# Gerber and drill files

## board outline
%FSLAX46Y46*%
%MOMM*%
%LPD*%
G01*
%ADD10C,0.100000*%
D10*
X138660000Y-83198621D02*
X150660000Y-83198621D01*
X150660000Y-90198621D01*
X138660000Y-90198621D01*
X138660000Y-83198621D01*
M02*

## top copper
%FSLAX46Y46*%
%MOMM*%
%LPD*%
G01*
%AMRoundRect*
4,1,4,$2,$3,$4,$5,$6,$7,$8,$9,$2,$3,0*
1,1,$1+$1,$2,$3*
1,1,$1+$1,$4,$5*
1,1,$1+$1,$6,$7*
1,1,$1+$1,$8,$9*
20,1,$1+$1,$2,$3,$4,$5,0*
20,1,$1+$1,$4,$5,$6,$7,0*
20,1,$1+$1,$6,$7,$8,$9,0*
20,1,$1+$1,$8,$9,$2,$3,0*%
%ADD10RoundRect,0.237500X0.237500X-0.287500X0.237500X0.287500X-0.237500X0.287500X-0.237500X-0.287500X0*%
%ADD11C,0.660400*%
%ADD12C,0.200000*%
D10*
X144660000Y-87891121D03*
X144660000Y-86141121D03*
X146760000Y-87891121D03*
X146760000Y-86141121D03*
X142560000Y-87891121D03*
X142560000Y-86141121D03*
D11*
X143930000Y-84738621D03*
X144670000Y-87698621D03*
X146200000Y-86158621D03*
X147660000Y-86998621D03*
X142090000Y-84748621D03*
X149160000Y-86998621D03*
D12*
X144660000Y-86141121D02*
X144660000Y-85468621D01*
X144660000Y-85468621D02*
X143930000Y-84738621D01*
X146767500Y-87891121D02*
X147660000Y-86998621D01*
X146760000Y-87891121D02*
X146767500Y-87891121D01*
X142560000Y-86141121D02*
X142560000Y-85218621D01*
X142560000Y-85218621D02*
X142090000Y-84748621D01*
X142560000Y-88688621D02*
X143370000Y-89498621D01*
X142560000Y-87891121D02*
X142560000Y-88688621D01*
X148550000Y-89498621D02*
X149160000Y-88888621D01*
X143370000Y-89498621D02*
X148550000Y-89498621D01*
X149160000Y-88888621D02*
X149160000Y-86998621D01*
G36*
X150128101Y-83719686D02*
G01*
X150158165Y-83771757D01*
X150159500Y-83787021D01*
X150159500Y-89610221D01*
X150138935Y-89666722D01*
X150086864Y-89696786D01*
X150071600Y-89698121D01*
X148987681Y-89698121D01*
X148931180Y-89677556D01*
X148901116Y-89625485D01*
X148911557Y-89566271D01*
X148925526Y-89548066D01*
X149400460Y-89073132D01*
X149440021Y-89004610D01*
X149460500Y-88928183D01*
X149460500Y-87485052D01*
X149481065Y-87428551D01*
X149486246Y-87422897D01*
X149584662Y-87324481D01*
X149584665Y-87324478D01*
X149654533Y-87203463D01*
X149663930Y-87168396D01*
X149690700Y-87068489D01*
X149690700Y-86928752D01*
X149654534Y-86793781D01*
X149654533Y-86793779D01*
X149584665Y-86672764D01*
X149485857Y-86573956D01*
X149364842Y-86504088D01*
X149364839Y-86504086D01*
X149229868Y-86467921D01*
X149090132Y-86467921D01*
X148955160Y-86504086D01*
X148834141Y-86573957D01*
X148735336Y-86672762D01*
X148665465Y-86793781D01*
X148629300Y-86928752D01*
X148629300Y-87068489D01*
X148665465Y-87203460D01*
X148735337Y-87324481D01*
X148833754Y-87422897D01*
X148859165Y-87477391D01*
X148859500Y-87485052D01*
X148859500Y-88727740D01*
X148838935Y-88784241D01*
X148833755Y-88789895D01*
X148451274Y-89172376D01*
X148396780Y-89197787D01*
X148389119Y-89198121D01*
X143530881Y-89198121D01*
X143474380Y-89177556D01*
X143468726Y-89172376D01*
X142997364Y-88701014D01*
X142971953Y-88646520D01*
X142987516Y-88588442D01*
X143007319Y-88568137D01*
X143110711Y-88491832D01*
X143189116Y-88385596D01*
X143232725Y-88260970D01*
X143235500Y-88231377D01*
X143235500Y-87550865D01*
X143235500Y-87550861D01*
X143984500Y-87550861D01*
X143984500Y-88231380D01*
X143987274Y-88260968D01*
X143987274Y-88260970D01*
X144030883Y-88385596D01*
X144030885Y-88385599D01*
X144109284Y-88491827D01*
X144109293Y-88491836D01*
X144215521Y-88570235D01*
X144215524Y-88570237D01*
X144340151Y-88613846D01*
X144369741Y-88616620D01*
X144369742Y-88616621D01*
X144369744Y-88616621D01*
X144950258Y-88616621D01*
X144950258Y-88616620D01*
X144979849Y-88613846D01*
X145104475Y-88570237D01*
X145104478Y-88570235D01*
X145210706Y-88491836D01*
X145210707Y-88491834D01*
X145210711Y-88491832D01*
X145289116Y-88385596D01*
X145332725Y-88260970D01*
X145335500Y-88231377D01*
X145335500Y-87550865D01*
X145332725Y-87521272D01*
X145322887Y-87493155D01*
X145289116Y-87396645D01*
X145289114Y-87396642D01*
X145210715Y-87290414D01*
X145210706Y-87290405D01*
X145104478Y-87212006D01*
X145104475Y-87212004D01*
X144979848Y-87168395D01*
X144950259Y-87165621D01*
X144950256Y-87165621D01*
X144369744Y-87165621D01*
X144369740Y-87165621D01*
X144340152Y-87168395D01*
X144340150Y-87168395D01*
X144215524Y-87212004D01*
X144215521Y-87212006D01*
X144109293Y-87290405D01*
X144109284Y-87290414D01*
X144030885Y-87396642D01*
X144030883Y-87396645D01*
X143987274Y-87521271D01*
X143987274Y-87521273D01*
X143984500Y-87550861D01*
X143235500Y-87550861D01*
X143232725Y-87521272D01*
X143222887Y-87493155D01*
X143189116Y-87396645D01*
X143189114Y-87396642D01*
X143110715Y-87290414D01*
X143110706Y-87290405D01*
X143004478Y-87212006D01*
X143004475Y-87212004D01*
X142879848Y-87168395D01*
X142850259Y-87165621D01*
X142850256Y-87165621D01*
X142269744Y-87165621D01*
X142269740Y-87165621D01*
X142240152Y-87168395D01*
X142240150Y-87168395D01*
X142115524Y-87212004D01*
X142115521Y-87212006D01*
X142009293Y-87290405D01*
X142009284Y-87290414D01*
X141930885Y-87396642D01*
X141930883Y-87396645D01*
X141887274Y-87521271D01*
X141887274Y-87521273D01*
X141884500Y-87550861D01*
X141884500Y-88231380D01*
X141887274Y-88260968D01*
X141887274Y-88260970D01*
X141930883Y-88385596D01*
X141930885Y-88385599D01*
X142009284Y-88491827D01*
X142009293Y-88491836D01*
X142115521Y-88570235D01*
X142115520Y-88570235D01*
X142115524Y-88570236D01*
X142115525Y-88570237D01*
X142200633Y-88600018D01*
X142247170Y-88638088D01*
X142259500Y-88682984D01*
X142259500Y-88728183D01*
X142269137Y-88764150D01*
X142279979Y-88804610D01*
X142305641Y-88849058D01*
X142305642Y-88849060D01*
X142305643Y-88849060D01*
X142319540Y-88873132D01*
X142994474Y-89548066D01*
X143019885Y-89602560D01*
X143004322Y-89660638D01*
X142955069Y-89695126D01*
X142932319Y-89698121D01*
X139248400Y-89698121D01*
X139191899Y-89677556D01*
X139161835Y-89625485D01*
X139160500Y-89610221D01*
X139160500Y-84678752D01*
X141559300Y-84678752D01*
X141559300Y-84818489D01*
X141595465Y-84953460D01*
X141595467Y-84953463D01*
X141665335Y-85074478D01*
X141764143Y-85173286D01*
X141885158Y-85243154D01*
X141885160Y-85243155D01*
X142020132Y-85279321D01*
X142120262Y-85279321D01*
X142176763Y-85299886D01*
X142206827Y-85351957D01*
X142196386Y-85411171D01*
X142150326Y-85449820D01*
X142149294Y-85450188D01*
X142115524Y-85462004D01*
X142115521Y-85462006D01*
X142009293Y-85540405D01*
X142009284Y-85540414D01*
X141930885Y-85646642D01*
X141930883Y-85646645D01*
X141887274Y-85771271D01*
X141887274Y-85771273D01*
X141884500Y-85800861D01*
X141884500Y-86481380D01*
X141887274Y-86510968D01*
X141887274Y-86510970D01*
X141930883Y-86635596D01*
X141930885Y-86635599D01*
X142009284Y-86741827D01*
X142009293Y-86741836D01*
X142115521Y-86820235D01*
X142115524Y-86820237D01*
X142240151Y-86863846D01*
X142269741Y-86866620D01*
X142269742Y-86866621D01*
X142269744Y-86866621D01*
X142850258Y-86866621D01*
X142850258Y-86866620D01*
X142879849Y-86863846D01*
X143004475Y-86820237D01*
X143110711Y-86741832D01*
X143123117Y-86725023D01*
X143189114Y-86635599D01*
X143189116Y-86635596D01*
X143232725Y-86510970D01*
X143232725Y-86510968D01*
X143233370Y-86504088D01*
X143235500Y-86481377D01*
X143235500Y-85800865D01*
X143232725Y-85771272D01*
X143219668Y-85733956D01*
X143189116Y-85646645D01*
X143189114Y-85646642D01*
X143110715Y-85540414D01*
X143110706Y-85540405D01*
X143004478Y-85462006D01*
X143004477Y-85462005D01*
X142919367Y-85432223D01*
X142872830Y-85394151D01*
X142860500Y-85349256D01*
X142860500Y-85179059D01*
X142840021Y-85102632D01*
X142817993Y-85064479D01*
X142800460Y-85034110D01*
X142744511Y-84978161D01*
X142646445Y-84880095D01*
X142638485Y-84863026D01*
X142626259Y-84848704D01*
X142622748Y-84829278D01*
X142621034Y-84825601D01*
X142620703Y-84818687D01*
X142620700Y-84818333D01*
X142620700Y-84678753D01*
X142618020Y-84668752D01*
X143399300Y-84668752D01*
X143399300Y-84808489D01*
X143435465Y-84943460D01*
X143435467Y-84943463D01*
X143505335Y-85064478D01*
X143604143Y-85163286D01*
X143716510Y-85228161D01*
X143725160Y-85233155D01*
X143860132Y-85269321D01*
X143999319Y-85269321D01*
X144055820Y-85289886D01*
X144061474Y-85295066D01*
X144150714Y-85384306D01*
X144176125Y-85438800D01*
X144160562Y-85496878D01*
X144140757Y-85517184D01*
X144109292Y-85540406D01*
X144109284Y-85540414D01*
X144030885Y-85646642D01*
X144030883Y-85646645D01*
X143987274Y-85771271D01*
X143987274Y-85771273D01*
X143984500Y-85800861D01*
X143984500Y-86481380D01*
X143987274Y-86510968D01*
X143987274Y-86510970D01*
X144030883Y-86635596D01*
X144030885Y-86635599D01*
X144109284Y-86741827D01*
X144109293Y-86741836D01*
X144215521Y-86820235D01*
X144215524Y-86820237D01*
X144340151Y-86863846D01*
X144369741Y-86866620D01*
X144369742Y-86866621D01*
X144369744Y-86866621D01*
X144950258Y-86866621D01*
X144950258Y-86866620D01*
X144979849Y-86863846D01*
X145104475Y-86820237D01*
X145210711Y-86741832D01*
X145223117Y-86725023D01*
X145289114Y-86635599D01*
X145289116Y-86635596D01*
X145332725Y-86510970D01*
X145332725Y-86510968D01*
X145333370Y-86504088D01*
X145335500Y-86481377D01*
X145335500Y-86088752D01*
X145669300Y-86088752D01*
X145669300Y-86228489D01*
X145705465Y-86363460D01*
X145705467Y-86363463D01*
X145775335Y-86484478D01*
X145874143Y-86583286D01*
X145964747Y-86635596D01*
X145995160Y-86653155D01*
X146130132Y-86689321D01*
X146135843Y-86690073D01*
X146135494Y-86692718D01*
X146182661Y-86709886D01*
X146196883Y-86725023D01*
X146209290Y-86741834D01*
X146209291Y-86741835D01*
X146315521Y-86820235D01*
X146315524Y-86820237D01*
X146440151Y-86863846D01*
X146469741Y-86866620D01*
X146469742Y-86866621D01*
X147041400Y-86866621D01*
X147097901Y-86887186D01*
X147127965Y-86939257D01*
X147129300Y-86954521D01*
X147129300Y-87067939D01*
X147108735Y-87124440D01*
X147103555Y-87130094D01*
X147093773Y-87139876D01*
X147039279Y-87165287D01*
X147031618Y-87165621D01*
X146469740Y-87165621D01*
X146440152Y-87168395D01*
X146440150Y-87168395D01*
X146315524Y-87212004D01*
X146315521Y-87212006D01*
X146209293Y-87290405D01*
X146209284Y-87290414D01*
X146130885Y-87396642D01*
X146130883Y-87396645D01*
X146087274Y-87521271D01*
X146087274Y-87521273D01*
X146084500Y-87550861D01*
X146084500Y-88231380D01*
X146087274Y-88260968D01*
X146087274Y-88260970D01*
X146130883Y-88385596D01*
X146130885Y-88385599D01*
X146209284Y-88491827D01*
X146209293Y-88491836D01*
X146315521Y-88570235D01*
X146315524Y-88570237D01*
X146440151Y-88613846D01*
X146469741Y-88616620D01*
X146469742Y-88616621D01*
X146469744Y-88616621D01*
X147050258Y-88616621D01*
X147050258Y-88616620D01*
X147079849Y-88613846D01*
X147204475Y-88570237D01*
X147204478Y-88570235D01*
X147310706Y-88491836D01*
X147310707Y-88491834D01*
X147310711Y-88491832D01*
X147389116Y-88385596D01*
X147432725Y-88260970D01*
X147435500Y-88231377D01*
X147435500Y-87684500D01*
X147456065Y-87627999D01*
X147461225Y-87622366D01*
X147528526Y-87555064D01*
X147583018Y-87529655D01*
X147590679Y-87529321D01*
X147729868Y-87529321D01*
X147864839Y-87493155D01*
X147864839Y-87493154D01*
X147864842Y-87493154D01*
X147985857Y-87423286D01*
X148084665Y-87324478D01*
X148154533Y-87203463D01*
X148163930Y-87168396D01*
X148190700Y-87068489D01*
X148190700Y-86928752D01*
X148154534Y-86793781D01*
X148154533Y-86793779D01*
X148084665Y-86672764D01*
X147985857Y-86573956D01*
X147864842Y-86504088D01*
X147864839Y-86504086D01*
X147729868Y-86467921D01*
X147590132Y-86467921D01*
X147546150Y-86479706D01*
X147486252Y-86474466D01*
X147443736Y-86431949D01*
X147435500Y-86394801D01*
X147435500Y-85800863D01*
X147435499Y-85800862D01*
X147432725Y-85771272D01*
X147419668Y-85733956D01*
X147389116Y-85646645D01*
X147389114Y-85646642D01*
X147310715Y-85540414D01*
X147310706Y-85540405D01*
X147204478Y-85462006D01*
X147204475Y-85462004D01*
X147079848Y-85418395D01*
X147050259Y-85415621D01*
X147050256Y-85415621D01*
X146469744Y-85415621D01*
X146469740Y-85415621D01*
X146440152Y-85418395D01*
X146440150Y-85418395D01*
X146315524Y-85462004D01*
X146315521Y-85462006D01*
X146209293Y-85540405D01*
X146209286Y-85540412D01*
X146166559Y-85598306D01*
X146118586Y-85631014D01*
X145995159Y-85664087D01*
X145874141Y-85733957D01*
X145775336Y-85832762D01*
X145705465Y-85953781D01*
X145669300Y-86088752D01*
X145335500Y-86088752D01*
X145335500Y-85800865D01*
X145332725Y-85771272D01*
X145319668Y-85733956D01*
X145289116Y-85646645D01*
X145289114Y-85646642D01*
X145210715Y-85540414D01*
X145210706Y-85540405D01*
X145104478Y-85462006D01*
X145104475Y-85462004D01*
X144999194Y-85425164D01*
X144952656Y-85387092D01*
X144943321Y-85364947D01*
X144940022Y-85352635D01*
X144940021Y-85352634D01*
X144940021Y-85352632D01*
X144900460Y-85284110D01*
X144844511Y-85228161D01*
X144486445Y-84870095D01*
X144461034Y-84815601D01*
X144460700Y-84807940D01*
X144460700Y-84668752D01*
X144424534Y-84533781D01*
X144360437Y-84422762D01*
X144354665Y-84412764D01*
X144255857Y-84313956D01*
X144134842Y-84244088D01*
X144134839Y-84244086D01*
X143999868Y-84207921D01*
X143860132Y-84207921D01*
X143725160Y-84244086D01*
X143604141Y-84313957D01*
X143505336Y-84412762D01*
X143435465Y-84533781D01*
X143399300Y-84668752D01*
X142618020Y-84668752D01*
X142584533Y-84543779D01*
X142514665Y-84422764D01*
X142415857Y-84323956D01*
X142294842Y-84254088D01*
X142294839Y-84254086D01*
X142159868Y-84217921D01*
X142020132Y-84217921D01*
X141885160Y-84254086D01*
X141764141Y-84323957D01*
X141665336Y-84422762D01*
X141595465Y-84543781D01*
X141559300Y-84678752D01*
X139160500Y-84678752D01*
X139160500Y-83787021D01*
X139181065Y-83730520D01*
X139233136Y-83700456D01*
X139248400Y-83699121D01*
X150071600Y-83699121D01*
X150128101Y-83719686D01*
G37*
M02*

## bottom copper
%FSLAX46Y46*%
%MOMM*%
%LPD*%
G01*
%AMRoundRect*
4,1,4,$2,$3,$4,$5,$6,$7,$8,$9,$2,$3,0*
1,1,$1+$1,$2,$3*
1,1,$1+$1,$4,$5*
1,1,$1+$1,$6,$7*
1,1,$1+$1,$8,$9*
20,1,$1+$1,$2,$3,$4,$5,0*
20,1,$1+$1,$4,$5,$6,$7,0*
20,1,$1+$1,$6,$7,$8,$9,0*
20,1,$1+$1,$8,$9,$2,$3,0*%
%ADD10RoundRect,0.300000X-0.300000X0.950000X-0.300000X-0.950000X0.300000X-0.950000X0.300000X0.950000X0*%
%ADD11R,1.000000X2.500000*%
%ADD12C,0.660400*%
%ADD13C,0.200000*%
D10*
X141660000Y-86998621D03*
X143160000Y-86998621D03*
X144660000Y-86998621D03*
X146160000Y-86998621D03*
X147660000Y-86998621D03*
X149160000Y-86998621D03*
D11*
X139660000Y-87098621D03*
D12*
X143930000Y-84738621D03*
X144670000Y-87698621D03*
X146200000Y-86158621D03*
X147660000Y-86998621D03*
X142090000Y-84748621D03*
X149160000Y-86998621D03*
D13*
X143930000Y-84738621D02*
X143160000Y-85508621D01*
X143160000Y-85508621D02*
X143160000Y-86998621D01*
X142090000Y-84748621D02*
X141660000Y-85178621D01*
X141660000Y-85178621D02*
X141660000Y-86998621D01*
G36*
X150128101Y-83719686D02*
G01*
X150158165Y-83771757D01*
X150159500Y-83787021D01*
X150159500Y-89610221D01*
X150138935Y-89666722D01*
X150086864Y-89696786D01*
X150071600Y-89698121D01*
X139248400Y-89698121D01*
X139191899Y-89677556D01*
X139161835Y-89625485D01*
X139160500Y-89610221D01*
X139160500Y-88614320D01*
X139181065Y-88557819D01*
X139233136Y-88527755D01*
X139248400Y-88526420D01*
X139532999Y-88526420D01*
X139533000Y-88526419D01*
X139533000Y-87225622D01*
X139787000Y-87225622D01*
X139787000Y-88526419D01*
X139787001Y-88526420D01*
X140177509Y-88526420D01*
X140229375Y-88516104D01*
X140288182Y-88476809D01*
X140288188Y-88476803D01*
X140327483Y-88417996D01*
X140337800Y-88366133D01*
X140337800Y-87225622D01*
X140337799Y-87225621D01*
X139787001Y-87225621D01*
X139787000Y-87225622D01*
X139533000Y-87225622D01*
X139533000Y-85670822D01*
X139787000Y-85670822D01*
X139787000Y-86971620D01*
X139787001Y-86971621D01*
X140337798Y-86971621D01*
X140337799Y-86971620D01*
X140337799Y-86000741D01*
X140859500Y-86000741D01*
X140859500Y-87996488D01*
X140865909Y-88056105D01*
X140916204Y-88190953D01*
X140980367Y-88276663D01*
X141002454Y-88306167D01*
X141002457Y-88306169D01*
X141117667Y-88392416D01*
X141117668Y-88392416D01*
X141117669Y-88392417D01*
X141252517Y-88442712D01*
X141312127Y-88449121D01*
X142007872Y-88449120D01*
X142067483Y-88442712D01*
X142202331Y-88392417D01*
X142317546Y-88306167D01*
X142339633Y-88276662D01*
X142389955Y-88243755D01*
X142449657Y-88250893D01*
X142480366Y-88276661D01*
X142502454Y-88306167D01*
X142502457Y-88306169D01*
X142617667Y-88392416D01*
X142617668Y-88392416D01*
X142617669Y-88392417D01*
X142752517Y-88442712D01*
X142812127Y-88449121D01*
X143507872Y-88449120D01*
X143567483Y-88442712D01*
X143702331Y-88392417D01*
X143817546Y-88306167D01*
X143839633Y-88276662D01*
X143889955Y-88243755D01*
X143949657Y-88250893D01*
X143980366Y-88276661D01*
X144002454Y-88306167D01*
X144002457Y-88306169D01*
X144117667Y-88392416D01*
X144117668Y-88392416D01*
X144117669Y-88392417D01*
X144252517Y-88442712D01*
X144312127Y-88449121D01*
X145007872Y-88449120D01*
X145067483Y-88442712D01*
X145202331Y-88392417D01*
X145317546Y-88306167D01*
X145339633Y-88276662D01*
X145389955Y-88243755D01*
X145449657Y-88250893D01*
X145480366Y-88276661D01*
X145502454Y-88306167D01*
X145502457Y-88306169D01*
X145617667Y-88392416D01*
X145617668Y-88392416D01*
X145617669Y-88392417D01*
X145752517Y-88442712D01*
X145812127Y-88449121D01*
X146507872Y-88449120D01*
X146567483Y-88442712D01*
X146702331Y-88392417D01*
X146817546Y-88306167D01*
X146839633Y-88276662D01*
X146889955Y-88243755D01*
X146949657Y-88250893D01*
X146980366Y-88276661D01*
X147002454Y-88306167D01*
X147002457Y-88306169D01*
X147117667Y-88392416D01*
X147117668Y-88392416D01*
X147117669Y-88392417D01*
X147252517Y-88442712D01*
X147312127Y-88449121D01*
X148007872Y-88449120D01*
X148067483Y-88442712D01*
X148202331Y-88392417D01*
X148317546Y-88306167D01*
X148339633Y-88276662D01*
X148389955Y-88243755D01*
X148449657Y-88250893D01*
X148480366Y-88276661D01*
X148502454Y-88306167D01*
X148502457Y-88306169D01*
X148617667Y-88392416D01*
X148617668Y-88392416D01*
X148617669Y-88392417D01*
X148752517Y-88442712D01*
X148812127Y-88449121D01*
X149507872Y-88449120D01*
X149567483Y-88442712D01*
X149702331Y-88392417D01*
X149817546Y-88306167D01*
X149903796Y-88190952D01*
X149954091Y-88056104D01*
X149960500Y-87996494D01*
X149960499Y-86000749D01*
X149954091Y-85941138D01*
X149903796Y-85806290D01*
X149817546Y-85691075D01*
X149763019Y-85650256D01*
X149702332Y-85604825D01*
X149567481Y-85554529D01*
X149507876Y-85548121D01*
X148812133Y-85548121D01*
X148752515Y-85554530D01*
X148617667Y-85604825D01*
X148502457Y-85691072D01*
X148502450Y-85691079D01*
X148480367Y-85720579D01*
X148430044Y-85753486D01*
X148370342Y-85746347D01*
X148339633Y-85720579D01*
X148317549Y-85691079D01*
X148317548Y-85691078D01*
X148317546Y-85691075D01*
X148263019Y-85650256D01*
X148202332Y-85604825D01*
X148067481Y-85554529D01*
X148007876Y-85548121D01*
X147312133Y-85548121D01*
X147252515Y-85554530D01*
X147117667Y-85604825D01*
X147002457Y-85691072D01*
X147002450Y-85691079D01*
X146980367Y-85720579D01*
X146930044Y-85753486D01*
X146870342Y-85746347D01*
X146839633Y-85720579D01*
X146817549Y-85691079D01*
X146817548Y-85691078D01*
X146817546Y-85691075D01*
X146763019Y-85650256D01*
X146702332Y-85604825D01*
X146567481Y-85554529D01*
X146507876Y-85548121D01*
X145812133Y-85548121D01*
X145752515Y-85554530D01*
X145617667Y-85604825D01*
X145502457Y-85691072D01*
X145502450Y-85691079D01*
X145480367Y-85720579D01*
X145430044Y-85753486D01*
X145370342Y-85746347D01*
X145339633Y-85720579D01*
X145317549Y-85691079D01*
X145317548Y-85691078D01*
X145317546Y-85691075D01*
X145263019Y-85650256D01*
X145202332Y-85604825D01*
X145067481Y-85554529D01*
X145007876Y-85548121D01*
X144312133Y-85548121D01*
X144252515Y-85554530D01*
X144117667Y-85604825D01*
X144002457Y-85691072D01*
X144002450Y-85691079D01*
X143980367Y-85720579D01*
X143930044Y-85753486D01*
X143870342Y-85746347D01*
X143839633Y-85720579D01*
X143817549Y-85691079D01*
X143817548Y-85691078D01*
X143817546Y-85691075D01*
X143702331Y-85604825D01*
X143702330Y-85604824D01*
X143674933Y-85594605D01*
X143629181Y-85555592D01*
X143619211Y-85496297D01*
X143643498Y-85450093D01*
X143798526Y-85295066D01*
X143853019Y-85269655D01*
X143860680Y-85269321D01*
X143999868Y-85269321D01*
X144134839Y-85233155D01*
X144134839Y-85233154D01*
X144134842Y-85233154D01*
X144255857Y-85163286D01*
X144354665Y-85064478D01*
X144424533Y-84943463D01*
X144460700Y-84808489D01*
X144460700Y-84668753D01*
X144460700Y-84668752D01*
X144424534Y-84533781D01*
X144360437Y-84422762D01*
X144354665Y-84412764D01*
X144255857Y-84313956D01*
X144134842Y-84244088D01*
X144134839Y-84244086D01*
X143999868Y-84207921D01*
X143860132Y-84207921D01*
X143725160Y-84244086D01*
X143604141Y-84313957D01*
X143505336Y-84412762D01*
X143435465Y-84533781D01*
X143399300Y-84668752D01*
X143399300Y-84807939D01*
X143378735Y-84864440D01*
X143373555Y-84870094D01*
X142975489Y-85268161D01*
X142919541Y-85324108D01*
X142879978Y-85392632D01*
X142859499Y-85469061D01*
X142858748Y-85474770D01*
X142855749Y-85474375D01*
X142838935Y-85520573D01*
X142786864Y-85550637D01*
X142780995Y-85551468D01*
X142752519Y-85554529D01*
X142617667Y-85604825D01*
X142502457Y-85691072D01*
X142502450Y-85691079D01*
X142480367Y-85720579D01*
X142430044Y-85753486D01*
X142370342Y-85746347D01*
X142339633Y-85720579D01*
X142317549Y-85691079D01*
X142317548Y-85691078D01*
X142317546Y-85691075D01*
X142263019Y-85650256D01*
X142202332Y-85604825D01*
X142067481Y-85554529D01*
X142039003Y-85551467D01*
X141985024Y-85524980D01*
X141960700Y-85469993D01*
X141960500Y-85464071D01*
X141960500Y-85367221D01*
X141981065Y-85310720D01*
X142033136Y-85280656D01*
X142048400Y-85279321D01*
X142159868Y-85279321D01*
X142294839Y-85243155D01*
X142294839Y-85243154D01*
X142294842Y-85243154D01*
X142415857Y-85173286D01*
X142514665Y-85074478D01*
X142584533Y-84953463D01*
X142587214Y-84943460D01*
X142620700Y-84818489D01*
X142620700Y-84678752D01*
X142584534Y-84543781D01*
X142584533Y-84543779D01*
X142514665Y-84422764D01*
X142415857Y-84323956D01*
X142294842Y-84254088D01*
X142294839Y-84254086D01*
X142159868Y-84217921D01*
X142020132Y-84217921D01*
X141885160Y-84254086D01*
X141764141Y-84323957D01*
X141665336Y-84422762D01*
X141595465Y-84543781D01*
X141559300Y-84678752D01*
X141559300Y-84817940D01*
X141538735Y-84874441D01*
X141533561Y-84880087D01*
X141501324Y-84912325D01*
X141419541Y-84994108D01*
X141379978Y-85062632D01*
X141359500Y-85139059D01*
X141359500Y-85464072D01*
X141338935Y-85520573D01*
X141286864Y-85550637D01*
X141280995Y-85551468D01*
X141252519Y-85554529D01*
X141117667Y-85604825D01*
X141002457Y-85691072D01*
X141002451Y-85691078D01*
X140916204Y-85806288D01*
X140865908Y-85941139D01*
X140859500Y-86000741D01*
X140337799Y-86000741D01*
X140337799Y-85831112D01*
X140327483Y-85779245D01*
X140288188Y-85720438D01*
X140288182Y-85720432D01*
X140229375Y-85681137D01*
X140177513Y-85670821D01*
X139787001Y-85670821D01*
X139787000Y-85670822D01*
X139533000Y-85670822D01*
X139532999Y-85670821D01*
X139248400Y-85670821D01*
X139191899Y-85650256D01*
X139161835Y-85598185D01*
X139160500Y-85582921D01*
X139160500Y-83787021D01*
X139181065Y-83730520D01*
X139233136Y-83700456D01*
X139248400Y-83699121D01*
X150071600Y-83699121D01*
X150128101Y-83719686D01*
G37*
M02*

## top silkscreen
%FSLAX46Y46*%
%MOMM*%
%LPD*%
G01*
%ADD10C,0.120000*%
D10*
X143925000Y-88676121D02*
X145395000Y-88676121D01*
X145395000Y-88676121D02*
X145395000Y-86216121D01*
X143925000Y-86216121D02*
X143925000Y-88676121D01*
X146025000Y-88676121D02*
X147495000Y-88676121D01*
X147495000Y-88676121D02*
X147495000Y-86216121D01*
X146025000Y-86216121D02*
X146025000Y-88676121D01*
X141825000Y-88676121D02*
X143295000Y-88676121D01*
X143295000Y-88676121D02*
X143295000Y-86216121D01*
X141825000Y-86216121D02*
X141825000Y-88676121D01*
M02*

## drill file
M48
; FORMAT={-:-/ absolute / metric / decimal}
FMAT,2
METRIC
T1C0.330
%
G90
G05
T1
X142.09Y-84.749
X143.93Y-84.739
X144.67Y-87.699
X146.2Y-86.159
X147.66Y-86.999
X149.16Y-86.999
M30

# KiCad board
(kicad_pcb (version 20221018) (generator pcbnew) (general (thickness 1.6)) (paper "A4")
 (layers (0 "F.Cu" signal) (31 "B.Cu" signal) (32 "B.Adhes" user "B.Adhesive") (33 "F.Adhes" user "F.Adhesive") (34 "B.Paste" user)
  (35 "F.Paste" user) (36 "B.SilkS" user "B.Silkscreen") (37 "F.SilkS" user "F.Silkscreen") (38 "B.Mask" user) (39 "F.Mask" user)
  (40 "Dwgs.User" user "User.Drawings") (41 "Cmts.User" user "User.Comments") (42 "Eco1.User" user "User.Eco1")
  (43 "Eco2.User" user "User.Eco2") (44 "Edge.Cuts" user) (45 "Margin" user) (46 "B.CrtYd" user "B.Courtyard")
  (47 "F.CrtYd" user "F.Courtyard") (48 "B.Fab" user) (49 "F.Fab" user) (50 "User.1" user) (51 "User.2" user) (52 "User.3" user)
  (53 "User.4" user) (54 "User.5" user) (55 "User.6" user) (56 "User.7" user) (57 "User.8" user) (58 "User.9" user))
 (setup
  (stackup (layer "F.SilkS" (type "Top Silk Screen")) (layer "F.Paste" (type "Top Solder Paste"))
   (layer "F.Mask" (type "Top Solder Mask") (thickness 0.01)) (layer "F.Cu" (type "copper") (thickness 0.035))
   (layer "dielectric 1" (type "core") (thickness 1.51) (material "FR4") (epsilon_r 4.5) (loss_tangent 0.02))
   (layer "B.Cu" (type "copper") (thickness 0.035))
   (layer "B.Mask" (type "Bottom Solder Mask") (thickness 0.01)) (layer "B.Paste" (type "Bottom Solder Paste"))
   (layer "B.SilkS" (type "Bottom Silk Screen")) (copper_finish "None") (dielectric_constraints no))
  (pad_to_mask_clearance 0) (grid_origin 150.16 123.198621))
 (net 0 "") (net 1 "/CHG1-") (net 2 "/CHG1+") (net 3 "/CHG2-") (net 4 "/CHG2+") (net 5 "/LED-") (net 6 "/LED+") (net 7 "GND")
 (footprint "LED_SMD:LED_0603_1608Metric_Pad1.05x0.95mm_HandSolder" (layer "F.Cu") (at 144.66 87.016121 90)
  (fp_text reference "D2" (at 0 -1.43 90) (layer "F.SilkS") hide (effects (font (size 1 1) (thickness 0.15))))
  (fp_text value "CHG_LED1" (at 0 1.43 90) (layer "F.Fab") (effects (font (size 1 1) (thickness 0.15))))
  (fp_line (start -1.66 -0.735) (end -1.66 0.735) (stroke (width 0.12) (type solid)) (layer "F.SilkS"))
  (fp_line (start -1.66 0.735) (end 0.8 0.735) (stroke (width 0.12) (type solid)) (layer "F.SilkS"))
  (fp_line (start 0.8 -0.735) (end -1.66 -0.735) (stroke (width 0.12) (type solid)) (layer "F.SilkS"))
  (pad "1" smd roundrect (at -0.875 0 90) (size 1.05 0.95) (layers "F.Cu" "F.Paste" "F.Mask") (roundrect_rratio 0.25) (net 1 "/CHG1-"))
  (pad "2" smd roundrect (at 0.875 0 90) (size 1.05 0.95) (layers "F.Cu" "F.Paste" "F.Mask") (roundrect_rratio 0.25) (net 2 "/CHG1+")))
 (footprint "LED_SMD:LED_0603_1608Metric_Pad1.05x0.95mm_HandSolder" (layer "F.Cu") (at 146.76 87.016121 90)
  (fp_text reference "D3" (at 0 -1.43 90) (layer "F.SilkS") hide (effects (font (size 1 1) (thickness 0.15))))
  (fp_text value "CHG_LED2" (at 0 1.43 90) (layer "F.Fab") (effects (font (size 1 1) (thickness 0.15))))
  (fp_line (start -1.66 -0.735) (end -1.66 0.735) (stroke (width 0.12) (type solid)) (layer "F.SilkS"))
  (fp_line (start -1.66 0.735) (end 0.8 0.735) (stroke (width 0.12) (type solid)) (layer "F.SilkS"))
  (fp_line (start 0.8 -0.735) (end -1.66 -0.735) (stroke (width 0.12) (type solid)) (layer "F.SilkS"))
  (pad "1" smd roundrect (at -0.875 0 90) (size 1.05 0.95) (layers "F.Cu" "F.Paste" "F.Mask") (roundrect_rratio 0.25) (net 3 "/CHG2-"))
  (pad "2" smd roundrect (at 0.875 0 90) (size 1.05 0.95) (layers "F.Cu" "F.Paste" "F.Mask") (roundrect_rratio 0.25) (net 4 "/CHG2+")))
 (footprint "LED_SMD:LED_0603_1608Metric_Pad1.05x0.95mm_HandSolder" (layer "F.Cu") (at 142.56 87.016121 90)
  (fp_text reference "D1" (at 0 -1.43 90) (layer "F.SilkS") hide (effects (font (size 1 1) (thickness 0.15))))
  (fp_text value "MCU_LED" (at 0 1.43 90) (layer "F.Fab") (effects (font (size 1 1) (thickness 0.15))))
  (fp_line (start -1.66 -0.735) (end -1.66 0.735) (stroke (width 0.12) (type solid)) (layer "F.SilkS"))
  (fp_line (start -1.66 0.735) (end 0.8 0.735) (stroke (width 0.12) (type solid)) (layer "F.SilkS"))
  (fp_line (start 0.8 -0.735) (end -1.66 -0.735) (stroke (width 0.12) (type solid)) (layer "F.SilkS"))
  (pad "1" smd roundrect (at -0.875 0 90) (size 1.05 0.95) (layers "F.Cu" "F.Paste" "F.Mask") (roundrect_rratio 0.25) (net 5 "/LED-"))
  (pad "2" smd roundrect (at 0.875 0 90) (size 1.05 0.95) (layers "F.Cu" "F.Paste" "F.Mask") (roundrect_rratio 0.25) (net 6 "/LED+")))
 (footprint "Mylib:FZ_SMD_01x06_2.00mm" (layer "B.Cu") (at 145.16 86.998621 -90)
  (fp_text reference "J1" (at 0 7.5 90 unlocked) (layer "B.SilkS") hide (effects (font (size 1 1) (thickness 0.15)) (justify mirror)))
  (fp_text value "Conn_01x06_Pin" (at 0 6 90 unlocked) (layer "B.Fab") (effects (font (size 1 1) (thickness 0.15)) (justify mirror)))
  (pad "1" smd roundrect (at 0 3.5 270) (size 2.5 1.2) (layers "B.Cu" "B.Paste" "B.Mask") (roundrect_rratio 0.25) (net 6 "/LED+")
   (thermal_bridge_angle 45))
  (pad "2" smd roundrect (at 0 2 270) (size 2.5 1.2) (layers "B.Cu" "B.Paste" "B.Mask") (roundrect_rratio 0.25) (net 2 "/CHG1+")
   (thermal_bridge_angle 45))
  (pad "3" smd roundrect (at 0 0.5 270) (size 2.5 1.2) (layers "B.Cu" "B.Paste" "B.Mask") (roundrect_rratio 0.25) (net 1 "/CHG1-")
   (thermal_bridge_angle 45))
  (pad "4" smd roundrect (at 0 -1 270) (size 2.5 1.2) (layers "B.Cu" "B.Paste" "B.Mask") (roundrect_rratio 0.25) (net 4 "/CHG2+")
   (thermal_bridge_angle 45))
  (pad "5" smd roundrect (at 0 -2.5 270) (size 2.5 1.2) (layers "B.Cu" "B.Paste" "B.Mask") (roundrect_rratio 0.25) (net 3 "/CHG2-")
   (thermal_bridge_angle 45))
  (pad "6" smd roundrect (at 0 -4 270) (size 2.5 1.2) (layers "B.Cu" "B.Paste" "B.Mask") (roundrect_rratio 0.25) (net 5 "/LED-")
   (thermal_bridge_angle 45)))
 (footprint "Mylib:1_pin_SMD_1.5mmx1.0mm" (layer "B.Cu") (at 137.66 87.098621 -90)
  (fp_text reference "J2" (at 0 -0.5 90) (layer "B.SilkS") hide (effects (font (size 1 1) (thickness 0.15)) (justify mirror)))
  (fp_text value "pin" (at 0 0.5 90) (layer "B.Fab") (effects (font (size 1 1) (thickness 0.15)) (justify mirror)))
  (pad "1" smd rect (at 0 -2 270) (size 2.5 1) (layers "B.Cu" "B.Paste" "B.Mask") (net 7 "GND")))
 (gr_rect (start 138.66 83.198621) (end 150.66 90.198621) (stroke (width 0.1) (type default)) (fill none) (layer "Edge.Cuts"))
 (segment (start 144.66 86.141121) (end 144.66 85.468621) (width 0.2) (layer "F.Cu") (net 2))
 (segment (start 144.66 85.468621) (end 143.93 84.738621) (width 0.2) (layer "F.Cu") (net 2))
 (via (at 143.93 84.738621) (size 0.6604) (drill 0.3302) (layers "F.Cu" "B.Cu") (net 2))
 (segment (start 143.93 84.738621) (end 143.16 85.508621) (width 0.2) (layer "B.Cu") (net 2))
 (segment (start 143.16 85.508621) (end 143.16 86.998621) (width 0.2) (layer "B.Cu") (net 2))
 (via (at 144.67 87.698621) (size 0.6604) (drill 0.3302) (layers "F.Cu" "B.Cu") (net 1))
 (via (at 146.2 86.158621) (size 0.6604) (drill 0.3302) (layers "F.Cu" "B.Cu") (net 4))
 (segment (start 146.7675 87.891121) (end 147.66 86.998621) (width 0.2) (layer "F.Cu") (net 3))
 (segment (start 146.76 87.891121) (end 146.7675 87.891121) (width 0.2) (layer "F.Cu") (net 3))
 (via (at 147.66 86.998621) (size 0.6604) (drill 0.3302) (layers "F.Cu" "B.Cu") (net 3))
 (segment (start 142.56 86.141121) (end 142.56 85.218621) (width 0.2) (layer "F.Cu") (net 6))
 (segment (start 142.56 85.218621) (end 142.09 84.748621) (width 0.2) (layer "F.Cu") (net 6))
 (via (at 142.09 84.748621) (size 0.6604) (drill 0.3302) (layers "F.Cu" "B.Cu") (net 6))
 (segment (start 142.09 84.748621) (end 141.66 85.178621) (width 0.2) (layer "B.Cu") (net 6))
 (segment (start 141.66 85.178621) (end 141.66 86.998621) (width 0.2) (layer "B.Cu") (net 6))
 (segment (start 142.56 88.688621) (end 143.37 89.498621) (width 0.2) (layer "F.Cu") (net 5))
 (segment (start 142.56 87.891121) (end 142.56 88.688621) (width 0.2) (layer "F.Cu") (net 5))
 (segment (start 148.55 89.498621) (end 149.16 88.888621) (width 0.2) (layer "F.Cu") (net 5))
 (segment (start 143.37 89.498621) (end 148.55 89.498621) (width 0.2) (layer "F.Cu") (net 5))
 (segment (start 149.16 88.888621) (end 149.16 86.998621) (width 0.2) (layer "F.Cu") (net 5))
 (via (at 149.16 86.998621) (size 0.6604) (drill 0.3302) (layers "F.Cu" "B.Cu") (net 5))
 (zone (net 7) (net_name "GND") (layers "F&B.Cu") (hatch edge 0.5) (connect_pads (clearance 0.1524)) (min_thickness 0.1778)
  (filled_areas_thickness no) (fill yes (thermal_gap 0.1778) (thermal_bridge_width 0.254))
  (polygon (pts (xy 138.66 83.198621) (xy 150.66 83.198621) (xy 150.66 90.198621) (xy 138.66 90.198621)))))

